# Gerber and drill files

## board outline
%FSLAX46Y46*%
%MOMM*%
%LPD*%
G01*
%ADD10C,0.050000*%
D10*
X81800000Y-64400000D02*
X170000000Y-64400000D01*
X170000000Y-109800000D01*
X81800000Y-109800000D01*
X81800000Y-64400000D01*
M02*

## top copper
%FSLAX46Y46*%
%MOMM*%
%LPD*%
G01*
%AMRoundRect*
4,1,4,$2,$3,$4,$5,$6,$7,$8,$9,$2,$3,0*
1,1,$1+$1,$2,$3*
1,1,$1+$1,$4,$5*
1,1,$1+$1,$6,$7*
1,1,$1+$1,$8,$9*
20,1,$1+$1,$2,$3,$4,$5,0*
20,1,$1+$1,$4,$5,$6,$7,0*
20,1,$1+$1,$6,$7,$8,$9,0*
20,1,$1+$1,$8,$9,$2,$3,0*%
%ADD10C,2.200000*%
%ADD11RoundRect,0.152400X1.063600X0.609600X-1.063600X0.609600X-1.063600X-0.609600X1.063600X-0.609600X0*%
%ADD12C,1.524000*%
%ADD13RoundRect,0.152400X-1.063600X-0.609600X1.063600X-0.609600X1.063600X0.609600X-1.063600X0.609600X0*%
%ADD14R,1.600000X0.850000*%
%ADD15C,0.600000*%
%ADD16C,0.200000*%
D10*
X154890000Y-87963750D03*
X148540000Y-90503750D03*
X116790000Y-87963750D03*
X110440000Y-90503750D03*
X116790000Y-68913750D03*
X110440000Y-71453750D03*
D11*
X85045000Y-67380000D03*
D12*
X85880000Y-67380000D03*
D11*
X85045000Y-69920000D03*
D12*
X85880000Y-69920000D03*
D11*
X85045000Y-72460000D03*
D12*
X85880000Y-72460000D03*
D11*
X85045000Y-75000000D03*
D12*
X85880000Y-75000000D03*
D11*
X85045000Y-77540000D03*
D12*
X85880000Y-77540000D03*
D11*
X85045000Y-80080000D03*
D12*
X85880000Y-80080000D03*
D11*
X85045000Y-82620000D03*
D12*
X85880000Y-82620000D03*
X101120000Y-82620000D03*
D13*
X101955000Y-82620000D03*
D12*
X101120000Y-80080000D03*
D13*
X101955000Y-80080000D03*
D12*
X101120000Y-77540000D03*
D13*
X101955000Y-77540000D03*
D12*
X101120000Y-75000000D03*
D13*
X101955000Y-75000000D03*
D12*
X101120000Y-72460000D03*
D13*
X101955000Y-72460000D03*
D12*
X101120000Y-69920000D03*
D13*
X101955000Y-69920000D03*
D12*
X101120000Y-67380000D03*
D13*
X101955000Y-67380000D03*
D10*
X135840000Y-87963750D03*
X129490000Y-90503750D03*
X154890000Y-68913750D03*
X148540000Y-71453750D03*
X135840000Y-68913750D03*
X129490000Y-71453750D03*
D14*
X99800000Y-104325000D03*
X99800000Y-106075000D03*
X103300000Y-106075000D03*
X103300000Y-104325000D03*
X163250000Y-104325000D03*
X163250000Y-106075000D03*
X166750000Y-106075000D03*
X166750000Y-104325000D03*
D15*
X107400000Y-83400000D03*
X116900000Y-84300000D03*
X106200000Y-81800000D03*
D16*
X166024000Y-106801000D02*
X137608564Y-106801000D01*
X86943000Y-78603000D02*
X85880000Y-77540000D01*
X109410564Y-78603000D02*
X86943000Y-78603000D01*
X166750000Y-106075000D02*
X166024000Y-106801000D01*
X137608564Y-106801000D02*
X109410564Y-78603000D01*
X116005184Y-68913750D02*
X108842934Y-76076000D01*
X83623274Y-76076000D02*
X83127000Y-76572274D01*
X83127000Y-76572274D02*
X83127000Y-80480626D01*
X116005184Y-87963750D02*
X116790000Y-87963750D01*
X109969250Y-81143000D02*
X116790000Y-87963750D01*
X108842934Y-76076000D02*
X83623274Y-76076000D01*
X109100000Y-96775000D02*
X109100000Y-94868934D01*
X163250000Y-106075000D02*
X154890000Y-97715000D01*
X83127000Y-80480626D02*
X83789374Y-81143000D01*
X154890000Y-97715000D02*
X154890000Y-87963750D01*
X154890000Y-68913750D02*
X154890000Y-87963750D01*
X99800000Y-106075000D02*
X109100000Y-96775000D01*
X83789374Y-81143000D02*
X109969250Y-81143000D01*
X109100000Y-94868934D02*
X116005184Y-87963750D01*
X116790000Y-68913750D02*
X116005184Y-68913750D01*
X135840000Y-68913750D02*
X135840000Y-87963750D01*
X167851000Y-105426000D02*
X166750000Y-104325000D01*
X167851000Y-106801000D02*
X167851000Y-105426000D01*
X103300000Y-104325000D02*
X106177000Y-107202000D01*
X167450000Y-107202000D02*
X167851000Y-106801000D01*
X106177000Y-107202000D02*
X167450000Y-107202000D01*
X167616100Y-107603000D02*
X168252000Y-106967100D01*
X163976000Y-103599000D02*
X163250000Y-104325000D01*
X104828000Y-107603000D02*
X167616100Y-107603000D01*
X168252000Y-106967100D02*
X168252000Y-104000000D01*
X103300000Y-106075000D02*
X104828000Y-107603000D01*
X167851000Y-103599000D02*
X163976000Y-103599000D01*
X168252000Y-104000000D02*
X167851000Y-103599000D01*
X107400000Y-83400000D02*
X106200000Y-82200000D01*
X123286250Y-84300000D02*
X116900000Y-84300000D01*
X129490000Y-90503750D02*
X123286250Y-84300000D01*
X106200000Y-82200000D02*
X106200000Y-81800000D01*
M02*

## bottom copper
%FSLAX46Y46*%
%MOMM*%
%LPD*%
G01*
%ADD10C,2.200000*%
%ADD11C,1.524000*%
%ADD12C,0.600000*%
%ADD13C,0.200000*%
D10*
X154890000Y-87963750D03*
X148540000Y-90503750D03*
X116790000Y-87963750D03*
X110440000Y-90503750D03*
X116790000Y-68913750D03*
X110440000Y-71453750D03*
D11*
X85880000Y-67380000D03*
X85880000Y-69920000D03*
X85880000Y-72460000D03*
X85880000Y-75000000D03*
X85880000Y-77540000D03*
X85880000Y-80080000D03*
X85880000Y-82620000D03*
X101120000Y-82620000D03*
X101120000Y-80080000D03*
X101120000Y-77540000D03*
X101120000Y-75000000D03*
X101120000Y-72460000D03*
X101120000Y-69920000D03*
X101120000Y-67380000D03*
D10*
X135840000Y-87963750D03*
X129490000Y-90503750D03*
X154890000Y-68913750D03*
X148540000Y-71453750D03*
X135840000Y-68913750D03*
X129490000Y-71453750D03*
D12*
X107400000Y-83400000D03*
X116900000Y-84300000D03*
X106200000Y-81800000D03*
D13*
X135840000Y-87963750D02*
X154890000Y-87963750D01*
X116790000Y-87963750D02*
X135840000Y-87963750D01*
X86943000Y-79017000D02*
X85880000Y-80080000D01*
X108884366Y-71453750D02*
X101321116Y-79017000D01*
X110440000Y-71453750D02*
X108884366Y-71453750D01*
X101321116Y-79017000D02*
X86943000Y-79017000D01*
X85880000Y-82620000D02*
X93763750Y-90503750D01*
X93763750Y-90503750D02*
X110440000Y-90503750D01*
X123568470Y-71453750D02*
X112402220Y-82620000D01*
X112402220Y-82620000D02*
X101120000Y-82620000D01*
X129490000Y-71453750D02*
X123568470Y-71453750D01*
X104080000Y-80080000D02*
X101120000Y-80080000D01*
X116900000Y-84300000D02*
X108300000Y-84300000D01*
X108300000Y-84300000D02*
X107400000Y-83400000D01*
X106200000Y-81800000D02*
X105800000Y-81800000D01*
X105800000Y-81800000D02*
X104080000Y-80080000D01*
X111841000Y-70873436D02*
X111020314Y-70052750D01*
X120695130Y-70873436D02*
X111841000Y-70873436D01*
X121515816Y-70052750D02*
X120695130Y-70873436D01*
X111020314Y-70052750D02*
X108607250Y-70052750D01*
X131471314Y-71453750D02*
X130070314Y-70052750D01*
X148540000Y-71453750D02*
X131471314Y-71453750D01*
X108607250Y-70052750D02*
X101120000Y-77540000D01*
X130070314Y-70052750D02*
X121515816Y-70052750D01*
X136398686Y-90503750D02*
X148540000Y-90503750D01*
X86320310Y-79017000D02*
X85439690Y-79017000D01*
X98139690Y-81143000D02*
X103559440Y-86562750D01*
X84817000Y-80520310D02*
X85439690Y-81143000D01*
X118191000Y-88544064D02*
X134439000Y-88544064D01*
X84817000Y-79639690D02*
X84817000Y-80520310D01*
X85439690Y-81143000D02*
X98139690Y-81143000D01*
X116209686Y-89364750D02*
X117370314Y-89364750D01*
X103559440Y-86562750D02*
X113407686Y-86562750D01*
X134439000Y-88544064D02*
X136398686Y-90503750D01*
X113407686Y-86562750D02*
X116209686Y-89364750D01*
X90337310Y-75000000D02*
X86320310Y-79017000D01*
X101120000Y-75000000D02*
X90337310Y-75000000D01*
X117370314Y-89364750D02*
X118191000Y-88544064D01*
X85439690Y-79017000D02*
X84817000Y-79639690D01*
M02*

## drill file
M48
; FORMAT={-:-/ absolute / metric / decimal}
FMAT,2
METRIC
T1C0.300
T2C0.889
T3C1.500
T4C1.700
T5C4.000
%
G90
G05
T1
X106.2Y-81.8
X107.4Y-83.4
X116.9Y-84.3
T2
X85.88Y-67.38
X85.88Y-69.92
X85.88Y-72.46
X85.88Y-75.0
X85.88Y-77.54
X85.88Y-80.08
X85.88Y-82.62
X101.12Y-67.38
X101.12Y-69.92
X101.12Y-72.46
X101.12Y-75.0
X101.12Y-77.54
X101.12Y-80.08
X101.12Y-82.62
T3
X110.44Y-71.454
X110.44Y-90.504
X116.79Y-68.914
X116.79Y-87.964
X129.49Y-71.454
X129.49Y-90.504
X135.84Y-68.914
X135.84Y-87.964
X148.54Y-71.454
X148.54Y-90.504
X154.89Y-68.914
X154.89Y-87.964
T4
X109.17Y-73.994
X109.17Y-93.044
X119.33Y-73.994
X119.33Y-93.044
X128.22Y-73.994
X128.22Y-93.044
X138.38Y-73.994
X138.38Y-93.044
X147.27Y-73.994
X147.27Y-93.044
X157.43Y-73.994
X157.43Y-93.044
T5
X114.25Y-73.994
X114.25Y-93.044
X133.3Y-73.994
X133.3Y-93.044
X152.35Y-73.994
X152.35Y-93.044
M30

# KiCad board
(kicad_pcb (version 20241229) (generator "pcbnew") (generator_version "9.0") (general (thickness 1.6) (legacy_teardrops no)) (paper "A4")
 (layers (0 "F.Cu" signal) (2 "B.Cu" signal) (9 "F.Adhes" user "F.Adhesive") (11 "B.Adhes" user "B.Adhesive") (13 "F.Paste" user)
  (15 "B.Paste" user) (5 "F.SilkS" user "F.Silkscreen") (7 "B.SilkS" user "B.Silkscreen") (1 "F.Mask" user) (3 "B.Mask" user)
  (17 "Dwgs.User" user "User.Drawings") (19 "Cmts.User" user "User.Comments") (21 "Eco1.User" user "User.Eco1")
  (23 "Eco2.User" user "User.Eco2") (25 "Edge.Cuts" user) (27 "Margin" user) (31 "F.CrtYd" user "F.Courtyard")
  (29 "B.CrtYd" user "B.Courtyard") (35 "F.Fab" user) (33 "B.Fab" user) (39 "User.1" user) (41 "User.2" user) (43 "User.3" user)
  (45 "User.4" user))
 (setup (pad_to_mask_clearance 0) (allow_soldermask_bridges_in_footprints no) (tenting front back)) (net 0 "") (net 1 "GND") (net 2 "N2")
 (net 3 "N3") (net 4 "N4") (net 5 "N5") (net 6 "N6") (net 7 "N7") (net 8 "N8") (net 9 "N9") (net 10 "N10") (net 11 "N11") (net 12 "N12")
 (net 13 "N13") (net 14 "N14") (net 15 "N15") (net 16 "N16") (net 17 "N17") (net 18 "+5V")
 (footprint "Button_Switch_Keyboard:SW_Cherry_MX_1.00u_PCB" (layer "F.Cu") (at 154.89 87.96375)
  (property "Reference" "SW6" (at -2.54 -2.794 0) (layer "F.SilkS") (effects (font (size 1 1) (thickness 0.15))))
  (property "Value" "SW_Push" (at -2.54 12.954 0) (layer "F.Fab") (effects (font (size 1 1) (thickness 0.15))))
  (pad "" np_thru_hole circle (at -7.62 5.08) (size 1.7 1.7) (drill 1.7) (layers "*.Cu" "*.Mask"))
  (pad "" np_thru_hole circle (at -2.54 5.08) (size 4 4) (drill 4) (layers "*.Cu" "*.Mask"))
  (pad "" np_thru_hole circle (at 2.54 5.08) (size 1.7 1.7) (drill 1.7) (layers "*.Cu" "*.Mask"))
  (pad "1" thru_hole circle (at 0 0) (size 2.2 2.2) (drill 1.5) (layers "*.Cu" "*.Mask") (remove_unused_layers no) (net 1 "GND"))
  (pad "2" thru_hole circle (at -6.35 2.54) (size 2.2 2.2) (drill 1.5) (layers "*.Cu" "*.Mask") (remove_unused_layers no) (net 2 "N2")))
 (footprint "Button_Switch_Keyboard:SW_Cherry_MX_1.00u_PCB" (layer "F.Cu") (at 116.79 87.96375)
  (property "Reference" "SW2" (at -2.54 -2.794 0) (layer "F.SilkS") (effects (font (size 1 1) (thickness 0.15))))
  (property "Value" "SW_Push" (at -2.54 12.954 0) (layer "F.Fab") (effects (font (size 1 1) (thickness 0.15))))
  (pad "" np_thru_hole circle (at -7.62 5.08) (size 1.7 1.7) (drill 1.7) (layers "*.Cu" "*.Mask"))
  (pad "" np_thru_hole circle (at -2.54 5.08) (size 4 4) (drill 4) (layers "*.Cu" "*.Mask"))
  (pad "" np_thru_hole circle (at 2.54 5.08) (size 1.7 1.7) (drill 1.7) (layers "*.Cu" "*.Mask"))
  (pad "1" thru_hole circle (at 0 0) (size 2.2 2.2) (drill 1.5) (layers "*.Cu" "*.Mask") (remove_unused_layers no) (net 1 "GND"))
  (pad "2" thru_hole circle (at -6.35 2.54) (size 2.2 2.2) (drill 1.5) (layers "*.Cu" "*.Mask") (remove_unused_layers no) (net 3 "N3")))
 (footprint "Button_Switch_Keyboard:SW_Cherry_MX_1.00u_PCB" (layer "F.Cu") (at 116.79 68.91375)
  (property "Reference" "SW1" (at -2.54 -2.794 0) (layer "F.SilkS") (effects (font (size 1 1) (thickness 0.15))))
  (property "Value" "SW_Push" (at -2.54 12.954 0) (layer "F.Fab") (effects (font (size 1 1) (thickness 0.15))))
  (pad "" np_thru_hole circle (at -7.62 5.08) (size 1.7 1.7) (drill 1.7) (layers "*.Cu" "*.Mask"))
  (pad "" np_thru_hole circle (at -2.54 5.08) (size 4 4) (drill 4) (layers "*.Cu" "*.Mask"))
  (pad "" np_thru_hole circle (at 2.54 5.08) (size 1.7 1.7) (drill 1.7) (layers "*.Cu" "*.Mask"))
  (pad "1" thru_hole circle (at 0 0) (size 2.2 2.2) (drill 1.5) (layers "*.Cu" "*.Mask") (remove_unused_layers no) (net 1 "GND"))
  (pad "2" thru_hole circle (at -6.35 2.54) (size 2.2 2.2) (drill 1.5) (layers "*.Cu" "*.Mask") (remove_unused_layers no) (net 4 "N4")))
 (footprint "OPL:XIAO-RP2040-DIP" (layer "F.Cu") (at 93.5 75)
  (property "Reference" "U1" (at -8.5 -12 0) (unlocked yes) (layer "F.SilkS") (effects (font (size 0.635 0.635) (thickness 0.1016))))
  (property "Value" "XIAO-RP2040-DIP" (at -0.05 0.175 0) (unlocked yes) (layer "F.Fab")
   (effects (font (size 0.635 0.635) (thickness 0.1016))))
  (pad "1" smd roundrect (at -8.455 -7.62 180) (size 2.432 1.524) (layers "F.Cu" "F.Mask") (roundrect_rratio 0.1) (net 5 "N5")
   (thermal_bridge_angle 45))
  (pad "1" thru_hole circle (at -7.62 -7.62 180) (size 1.524 1.524) (drill 0.889) (layers "*.Cu" "*.Mask") (remove_unused_layers no)
   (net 5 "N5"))
  (pad "2" smd roundrect (at -8.455 -5.08 180) (size 2.432 1.524) (layers "F.Cu" "F.Mask") (roundrect_rratio 0.1) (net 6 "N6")
   (thermal_bridge_angle 45))
  (pad "2" thru_hole circle (at -7.62 -5.08 180) (size 1.524 1.524) (drill 0.889) (layers "*.Cu" "*.Mask") (remove_unused_layers no)
   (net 6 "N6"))
  (pad "3" smd roundrect (at -8.455 -2.54 180) (size 2.432 1.524) (layers "F.Cu" "F.Mask") (roundrect_rratio 0.1) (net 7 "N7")
   (thermal_bridge_angle 45))
  (pad "3" thru_hole circle (at -7.62 -2.54 180) (size 1.524 1.524) (drill 0.889) (layers "*.Cu" "*.Mask") (remove_unused_layers no)
   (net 7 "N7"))
  (pad "4" smd roundrect (at -8.455 0 180) (size 2.432 1.524) (layers "F.Cu" "F.Mask") (roundrect_rratio 0.1) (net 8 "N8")
   (thermal_bridge_angle 45))
  (pad "4" thru_hole circle (at -7.62 0 180) (size 1.524 1.524) (drill 0.889) (layers "*.Cu" "*.Mask") (remove_unused_layers no)
   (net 8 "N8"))
  (pad "5" smd roundrect (at -8.455 2.54 180) (size 2.432 1.524) (layers "F.Cu" "F.Mask") (roundrect_rratio 0.1) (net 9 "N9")
   (thermal_bridge_angle 45))
  (pad "5" thru_hole circle (at -7.62 2.54 180) (size 1.524 1.524) (drill 0.889) (layers "*.Cu" "*.Mask") (remove_unused_layers no)
   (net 9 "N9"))
  (pad "6" smd roundrect (at -8.455 5.08 180) (size 2.432 1.524) (layers "F.Cu" "F.Mask") (roundrect_rratio 0.1) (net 4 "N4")
   (thermal_bridge_angle 45))
  (pad "6" thru_hole circle (at -7.62 5.08 180) (size 1.524 1.524) (drill 0.889) (layers "*.Cu" "*.Mask") (remove_unused_layers no)
   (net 4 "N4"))
  (pad "7" smd roundrect (at -8.455 7.62 180) (size 2.432 1.524) (layers "F.Cu" "F.Mask") (roundrect_rratio 0.1) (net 3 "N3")
   (thermal_bridge_angle 45))
  (pad "7" thru_hole circle (at -7.62 7.62 180) (size 1.524 1.524) (drill 0.889) (layers "*.Cu" "*.Mask") (remove_unused_layers no)
   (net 3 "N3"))
  (pad "8" thru_hole circle (at 7.62 7.62) (size 1.524 1.524) (drill 0.889) (layers "*.Cu" "*.Mask") (remove_unused_layers no)
   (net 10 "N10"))
  (pad "8" smd roundrect (at 8.455 7.62) (size 2.432 1.524) (layers "F.Cu" "F.Mask") (roundrect_rratio 0.1) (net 10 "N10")
   (thermal_bridge_angle 45))
  (pad "9" thru_hole circle (at 7.62 5.08) (size 1.524 1.524) (drill 0.889) (layers "*.Cu" "*.Mask") (remove_unused_layers no)
   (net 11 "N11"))
  (pad "9" smd roundrect (at 8.455 5.08) (size 2.432 1.524) (layers "F.Cu" "F.Mask") (roundrect_rratio 0.1) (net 11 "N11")
   (thermal_bridge_angle 45))
  (pad "10" thru_hole circle (at 7.62 2.54) (size 1.524 1.524) (drill 0.889) (layers "*.Cu" "*.Mask") (remove_unused_layers no)
   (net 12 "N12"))
  (pad "10" smd roundrect (at 8.455 2.54) (size 2.432 1.524) (layers "F.Cu" "F.Mask") (roundrect_rratio 0.1) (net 12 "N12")
   (thermal_bridge_angle 45))
  (pad "11" thru_hole circle (at 7.62 0) (size 1.524 1.524) (drill 0.889) (layers "*.Cu" "*.Mask") (remove_unused_layers no) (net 2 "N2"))
  (pad "11" smd roundrect (at 8.455 0) (size 2.432 1.524) (layers "F.Cu" "F.Mask") (roundrect_rratio 0.1) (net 2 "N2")
   (thermal_bridge_angle 45))
  (pad "12" thru_hole circle (at 7.62 -2.54) (size 1.524 1.524) (drill 0.889) (layers "*.Cu" "*.Mask") (remove_unused_layers no)
   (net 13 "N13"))
  (pad "12" smd roundrect (at 8.455 -2.54) (size 2.432 1.524) (layers "F.Cu" "F.Mask") (roundrect_rratio 0.1) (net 13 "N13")
   (thermal_bridge_angle 45))
  (pad "13" thru_hole circle (at 7.62 -5.08) (size 1.524 1.524) (drill 0.889) (layers "*.Cu" "*.Mask") (remove_unused_layers no)
   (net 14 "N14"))
  (pad "13" smd roundrect (at 8.455 -5.08) (size 2.432 1.524) (layers "F.Cu" "F.Mask") (roundrect_rratio 0.1) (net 14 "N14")
   (thermal_bridge_angle 45))
  (pad "14" thru_hole circle (at 7.62 -7.62) (size 1.524 1.524) (drill 0.889) (layers "*.Cu" "*.Mask") (remove_unused_layers no)
   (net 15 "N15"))
  (pad "14" smd roundrect (at 8.455 -7.62) (size 2.432 1.524) (layers "F.Cu" "F.Mask") (roundrect_rratio 0.1) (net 15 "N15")
   (thermal_bridge_angle 45)))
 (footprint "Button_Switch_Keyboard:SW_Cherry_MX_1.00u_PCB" (layer "F.Cu") (at 135.84 87.96375)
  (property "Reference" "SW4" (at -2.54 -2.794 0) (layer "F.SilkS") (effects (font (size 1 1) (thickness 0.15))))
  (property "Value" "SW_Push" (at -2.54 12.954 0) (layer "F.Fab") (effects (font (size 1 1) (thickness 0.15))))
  (pad "" np_thru_hole circle (at -7.62 5.08) (size 1.7 1.7) (drill 1.7) (layers "*.Cu" "*.Mask"))
  (pad "" np_thru_hole circle (at -2.54 5.08) (size 4 4) (drill 4) (layers "*.Cu" "*.Mask"))
  (pad "" np_thru_hole circle (at 2.54 5.08) (size 1.7 1.7) (drill 1.7) (layers "*.Cu" "*.Mask"))
  (pad "1" thru_hole circle (at 0 0) (size 2.2 2.2) (drill 1.5) (layers "*.Cu" "*.Mask") (remove_unused_layers no) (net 1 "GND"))
  (pad "2" thru_hole circle (at -6.35 2.54) (size 2.2 2.2) (drill 1.5) (layers "*.Cu" "*.Mask") (remove_unused_layers no) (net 11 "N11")))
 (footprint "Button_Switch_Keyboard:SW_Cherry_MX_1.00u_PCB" (layer "F.Cu") (at 154.89 68.91375)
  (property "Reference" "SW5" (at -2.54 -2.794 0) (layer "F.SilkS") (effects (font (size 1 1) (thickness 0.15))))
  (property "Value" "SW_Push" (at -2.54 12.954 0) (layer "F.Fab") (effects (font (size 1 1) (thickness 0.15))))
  (pad "" np_thru_hole circle (at -7.62 5.08) (size 1.7 1.7) (drill 1.7) (layers "*.Cu" "*.Mask"))
  (pad "" np_thru_hole circle (at -2.54 5.08) (size 4 4) (drill 4) (layers "*.Cu" "*.Mask"))
  (pad "" np_thru_hole circle (at 2.54 5.08) (size 1.7 1.7) (drill 1.7) (layers "*.Cu" "*.Mask"))
  (pad "1" thru_hole circle (at 0 0) (size 2.2 2.2) (drill 1.5) (layers "*.Cu" "*.Mask") (remove_unused_layers no) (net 1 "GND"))
  (pad "2" thru_hole circle (at -6.35 2.54) (size 2.2 2.2) (drill 1.5) (layers "*.Cu" "*.Mask") (remove_unused_layers no) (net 12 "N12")))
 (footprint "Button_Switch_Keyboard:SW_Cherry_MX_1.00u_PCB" (layer "F.Cu") (at 135.84 68.91375)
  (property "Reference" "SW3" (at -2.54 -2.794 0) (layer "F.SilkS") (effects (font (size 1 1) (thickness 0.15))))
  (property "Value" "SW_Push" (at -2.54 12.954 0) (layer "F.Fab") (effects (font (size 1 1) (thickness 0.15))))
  (pad "" np_thru_hole circle (at -7.62 5.08) (size 1.7 1.7) (drill 1.7) (layers "*.Cu" "*.Mask"))
  (pad "" np_thru_hole circle (at -2.54 5.08) (size 4 4) (drill 4) (layers "*.Cu" "*.Mask"))
  (pad "" np_thru_hole circle (at 2.54 5.08) (size 1.7 1.7) (drill 1.7) (layers "*.Cu" "*.Mask"))
  (pad "1" thru_hole circle (at 0 0) (size 2.2 2.2) (drill 1.5) (layers "*.Cu" "*.Mask") (remove_unused_layers no) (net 1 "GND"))
  (pad "2" thru_hole circle (at -6.35 2.54) (size 2.2 2.2) (drill 1.5) (layers "*.Cu" "*.Mask") (remove_unused_layers no) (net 10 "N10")))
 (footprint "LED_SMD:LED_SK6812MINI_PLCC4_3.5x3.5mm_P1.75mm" (layer "F.Cu") (at 101.55 105.2)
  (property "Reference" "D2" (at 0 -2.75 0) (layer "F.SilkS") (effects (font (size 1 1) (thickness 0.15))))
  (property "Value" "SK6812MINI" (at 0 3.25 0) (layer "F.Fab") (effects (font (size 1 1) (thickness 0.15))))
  (pad "1" smd rect (at -1.75 -0.875) (size 1.6 0.85) (layers "F.Cu" "F.Mask" "F.Paste") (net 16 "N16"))
  (pad "2" smd rect (at -1.75 0.875) (size 1.6 0.85) (layers "F.Cu" "F.Mask" "F.Paste") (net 1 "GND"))
  (pad "3" smd rect (at 1.75 0.875) (size 1.6 0.85) (layers "F.Cu" "F.Mask" "F.Paste") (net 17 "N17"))
  (pad "4" smd rect (at 1.75 -0.875) (size 1.6 0.85) (layers "F.Cu" "F.Mask" "F.Paste") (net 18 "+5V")))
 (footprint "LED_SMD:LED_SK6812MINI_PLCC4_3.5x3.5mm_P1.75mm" (layer "F.Cu") (at 165 105.2)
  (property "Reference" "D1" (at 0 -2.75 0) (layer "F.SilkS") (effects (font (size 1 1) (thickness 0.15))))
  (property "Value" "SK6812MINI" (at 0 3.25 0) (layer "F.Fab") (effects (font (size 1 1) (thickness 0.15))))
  (pad "1" smd rect (at -1.75 -0.875) (size 1.6 0.85) (layers "F.Cu" "F.Mask" "F.Paste") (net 17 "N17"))
  (pad "2" smd rect (at -1.75 0.875) (size 1.6 0.85) (layers "F.Cu" "F.Mask" "F.Paste") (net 1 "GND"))
  (pad "3" smd rect (at 1.75 0.875) (size 1.6 0.85) (layers "F.Cu" "F.Mask" "F.Paste") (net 9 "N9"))
  (pad "4" smd rect (at 1.75 -0.875) (size 1.6 0.85) (layers "F.Cu" "F.Mask" "F.Paste") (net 18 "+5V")))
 (gr_rect (start 81.8 64.4) (end 170 109.8) (stroke (width 0.05) (type default)) (fill no) (layer "Edge.Cuts"))
 (segment (start 166.024 106.801) (end 137.608564 106.801) (width 0.2) (layer "F.Cu") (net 9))
 (segment (start 86.943 78.603) (end 85.88 77.54) (width 0.2) (layer "F.Cu") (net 9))
 (segment (start 109.410564 78.603) (end 86.943 78.603) (width 0.2) (layer "F.Cu") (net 9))
 (segment (start 166.75 106.075) (end 166.024 106.801) (width 0.2) (layer "F.Cu") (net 9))
 (segment (start 137.608564 106.801) (end 109.410564 78.603) (width 0.2) (layer "F.Cu") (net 9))
 (segment (start 116.005184 68.91375) (end 108.842934 76.076) (width 0.2) (layer "F.Cu") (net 1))
 (segment (start 83.623274 76.076) (end 83.127 76.572274) (width 0.2) (layer "F.Cu") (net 1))
 (segment (start 83.127 76.572274) (end 83.127 80.480626) (width 0.2) (layer "F.Cu") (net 1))
 (segment (start 116.005184 87.96375) (end 116.79 87.96375) (width 0.2) (layer "F.Cu") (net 1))
 (segment (start 109.96925 81.143) (end 116.79 87.96375) (width 0.2) (layer "F.Cu") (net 1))
 (segment (start 108.842934 76.076) (end 83.623274 76.076) (width 0.2) (layer "F.Cu") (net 1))
 (segment (start 109.1 96.775) (end 109.1 94.868934) (width 0.2) (layer "F.Cu") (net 1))
 (segment (start 163.25 106.075) (end 154.89 97.715) (width 0.2) (layer "F.Cu") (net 1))
 (segment (start 83.127 80.480626) (end 83.789374 81.143) (width 0.2) (layer "F.Cu") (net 1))
 (segment (start 154.89 97.715) (end 154.89 87.96375) (width 0.2) (layer "F.Cu") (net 1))
 (segment (start 154.89 68.91375) (end 154.89 87.96375) (width 0.2) (layer "F.Cu") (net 1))
 (segment (start 99.8 106.075) (end 109.1 96.775) (width 0.2) (layer "F.Cu") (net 1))
 (segment (start 83.789374 81.143) (end 109.96925 81.143) (width 0.2) (layer "F.Cu") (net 1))
 (segment (start 109.1 94.868934) (end 116.005184 87.96375) (width 0.2) (layer "F.Cu") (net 1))
 (segment (start 116.79 68.91375) (end 116.005184 68.91375) (width 0.2) (layer "F.Cu") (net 1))
 (segment (start 135.84 68.91375) (end 135.84 87.96375) (width 0.2) (layer "F.Cu") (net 1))
 (segment (start 135.84 87.96375) (end 154.89 87.96375) (width 0.2) (layer "B.Cu") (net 1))
 (segment (start 116.79 87.96375) (end 135.84 87.96375) (width 0.2) (layer "B.Cu") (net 1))
 (segment (start 167.851 105.426) (end 166.75 104.325) (width 0.2) (layer "F.Cu") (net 18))
 (segment (start 167.851 106.801) (end 167.851 105.426) (width 0.2) (layer "F.Cu") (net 18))
 (segment (start 103.3 104.325) (end 106.177 107.202) (width 0.2) (layer "F.Cu") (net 18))
 (segment (start 167.45 107.202) (end 167.851 106.801) (width 0.2) (layer "F.Cu") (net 18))
 (segment (start 106.177 107.202) (end 167.45 107.202) (width 0.2) (layer "F.Cu") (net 18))
 (segment (start 167.6161 107.603) (end 168.252 106.9671) (width 0.2) (layer "F.Cu") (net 17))
 (segment (start 163.976 103.599) (end 163.25 104.325) (width 0.2) (layer "F.Cu") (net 17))
 (segment (start 104.828 107.603) (end 167.6161 107.603) (width 0.2) (layer "F.Cu") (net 17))
 (segment (start 168.252 106.9671) (end 168.252 104) (width 0.2) (layer "F.Cu") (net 17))
 (segment (start 103.3 106.075) (end 104.828 107.603) (width 0.2) (layer "F.Cu") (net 17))
 (segment (start 167.851 103.599) (end 163.976 103.599) (width 0.2) (layer "F.Cu") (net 17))
 (segment (start 168.252 104) (end 167.851 103.599) (width 0.2) (layer "F.Cu") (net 17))
 (segment (start 86.943 79.017) (end 85.88 80.08) (width 0.2) (layer "B.Cu") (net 4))
 (segment (start 108.884366 71.45375) (end 101.321116 79.017) (width 0.2) (layer "B.Cu") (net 4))
 (segment (start 110.44 71.45375) (end 108.884366 71.45375) (width 0.2) (layer "B.Cu") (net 4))
 (segment (start 101.321116 79.017) (end 86.943 79.017) (width 0.2) (layer "B.Cu") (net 4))
 (segment (start 85.88 82.62) (end 93.76375 90.50375) (width 0.2) (layer "B.Cu") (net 3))
 (segment (start 93.76375 90.50375) (end 110.44 90.50375) (width 0.2) (layer "B.Cu") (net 3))
 (segment (start 123.56847 71.45375) (end 112.40222 82.62) (width 0.2) (layer "B.Cu") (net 10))
 (segment (start 112.40222 82.62) (end 101.12 82.62) (width 0.2) (layer "B.Cu") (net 10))
 (segment (start 129.49 71.45375) (end 123.56847 71.45375) (width 0.2) (layer "B.Cu") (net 10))
 (segment (start 107.4 83.4) (end 106.2 82.2) (width 0.2) (layer "F.Cu") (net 11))
 (segment (start 123.28625 84.3) (end 116.9 84.3) (width 0.2) (layer "F.Cu") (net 11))
 (segment (start 129.49 90.50375) (end 123.28625 84.3) (width 0.2) (layer "F.Cu") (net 11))
 (segment (start 106.2 82.2) (end 106.2 81.8) (width 0.2) (layer "F.Cu") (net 11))
 (via (at 107.4 83.4) (size 0.6) (drill 0.3) (layers "F.Cu" "B.Cu") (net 11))
 (via (at 116.9 84.3) (size 0.6) (drill 0.3) (layers "F.Cu" "B.Cu") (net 11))
 (via (at 106.2 81.8) (size 0.6) (drill 0.3) (layers "F.Cu" "B.Cu") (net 11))
 (segment (start 104.08 80.08) (end 101.12 80.08) (width 0.2) (layer "B.Cu") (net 11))
 (segment (start 116.9 84.3) (end 108.3 84.3) (width 0.2) (layer "B.Cu") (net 11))
 (segment (start 108.3 84.3) (end 107.4 83.4) (width 0.2) (layer "B.Cu") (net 11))
 (segment (start 106.2 81.8) (end 105.8 81.8) (width 0.2) (layer "B.Cu") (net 11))
 (segment (start 105.8 81.8) (end 104.08 80.08) (width 0.2) (layer "B.Cu") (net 11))
 (segment (start 111.841 70.873436) (end 111.020314 70.05275) (width 0.2) (layer "B.Cu") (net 12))
 (segment (start 120.69513 70.873436) (end 111.841 70.873436) (width 0.2) (layer "B.Cu") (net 12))
 (segment (start 121.515816 70.05275) (end 120.69513 70.873436) (width 0.2) (layer "B.Cu") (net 12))
 (segment (start 111.020314 70.05275) (end 108.60725 70.05275) (width 0.2) (layer "B.Cu") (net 12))
 (segment (start 131.471314 71.45375) (end 130.070314 70.05275) (width 0.2) (layer "B.Cu") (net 12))
 (segment (start 148.54 71.45375) (end 131.471314 71.45375) (width 0.2) (layer "B.Cu") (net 12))
 (segment (start 108.60725 70.05275) (end 101.12 77.54) (width 0.2) (layer "B.Cu") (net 12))
 (segment (start 130.070314 70.05275) (end 121.515816 70.05275) (width 0.2) (layer "B.Cu") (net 12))
 (segment (start 136.398686 90.50375) (end 148.54 90.50375) (width 0.2) (layer "B.Cu") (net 2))
 (segment (start 86.32031 79.017) (end 85.43969 79.017) (width 0.2) (layer "B.Cu") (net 2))
 (segment (start 98.13969 81.143) (end 103.55944 86.56275) (width 0.2) (layer "B.Cu") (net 2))
 (segment (start 84.817 80.52031) (end 85.43969 81.143) (width 0.2) (layer "B.Cu") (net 2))
 (segment (start 118.191 88.544064) (end 134.439 88.544064) (width 0.2) (layer "B.Cu") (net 2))
 (segment (start 84.817 79.63969) (end 84.817 80.52031) (width 0.2) (layer "B.Cu") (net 2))
 (segment (start 85.43969 81.143) (end 98.13969 81.143) (width 0.2) (layer "B.Cu") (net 2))
 (segment (start 116.209686 89.36475) (end 117.370314 89.36475) (width 0.2) (layer "B.Cu") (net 2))
 (segment (start 103.55944 86.56275) (end 113.407686 86.56275) (width 0.2) (layer "B.Cu") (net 2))
 (segment (start 134.439 88.544064) (end 136.398686 90.50375) (width 0.2) (layer "B.Cu") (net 2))
 (segment (start 113.407686 86.56275) (end 116.209686 89.36475) (width 0.2) (layer "B.Cu") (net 2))
 (segment (start 90.33731 75) (end 86.32031 79.017) (width 0.2) (layer "B.Cu") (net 2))
 (segment (start 101.12 75) (end 90.33731 75) (width 0.2) (layer "B.Cu") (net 2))
 (segment (start 117.370314 89.36475) (end 118.191 88.544064) (width 0.2) (layer "B.Cu") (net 2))
 (segment (start 85.43969 79.017) (end 84.817 79.63969) (width 0.2) (layer "B.Cu") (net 2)))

